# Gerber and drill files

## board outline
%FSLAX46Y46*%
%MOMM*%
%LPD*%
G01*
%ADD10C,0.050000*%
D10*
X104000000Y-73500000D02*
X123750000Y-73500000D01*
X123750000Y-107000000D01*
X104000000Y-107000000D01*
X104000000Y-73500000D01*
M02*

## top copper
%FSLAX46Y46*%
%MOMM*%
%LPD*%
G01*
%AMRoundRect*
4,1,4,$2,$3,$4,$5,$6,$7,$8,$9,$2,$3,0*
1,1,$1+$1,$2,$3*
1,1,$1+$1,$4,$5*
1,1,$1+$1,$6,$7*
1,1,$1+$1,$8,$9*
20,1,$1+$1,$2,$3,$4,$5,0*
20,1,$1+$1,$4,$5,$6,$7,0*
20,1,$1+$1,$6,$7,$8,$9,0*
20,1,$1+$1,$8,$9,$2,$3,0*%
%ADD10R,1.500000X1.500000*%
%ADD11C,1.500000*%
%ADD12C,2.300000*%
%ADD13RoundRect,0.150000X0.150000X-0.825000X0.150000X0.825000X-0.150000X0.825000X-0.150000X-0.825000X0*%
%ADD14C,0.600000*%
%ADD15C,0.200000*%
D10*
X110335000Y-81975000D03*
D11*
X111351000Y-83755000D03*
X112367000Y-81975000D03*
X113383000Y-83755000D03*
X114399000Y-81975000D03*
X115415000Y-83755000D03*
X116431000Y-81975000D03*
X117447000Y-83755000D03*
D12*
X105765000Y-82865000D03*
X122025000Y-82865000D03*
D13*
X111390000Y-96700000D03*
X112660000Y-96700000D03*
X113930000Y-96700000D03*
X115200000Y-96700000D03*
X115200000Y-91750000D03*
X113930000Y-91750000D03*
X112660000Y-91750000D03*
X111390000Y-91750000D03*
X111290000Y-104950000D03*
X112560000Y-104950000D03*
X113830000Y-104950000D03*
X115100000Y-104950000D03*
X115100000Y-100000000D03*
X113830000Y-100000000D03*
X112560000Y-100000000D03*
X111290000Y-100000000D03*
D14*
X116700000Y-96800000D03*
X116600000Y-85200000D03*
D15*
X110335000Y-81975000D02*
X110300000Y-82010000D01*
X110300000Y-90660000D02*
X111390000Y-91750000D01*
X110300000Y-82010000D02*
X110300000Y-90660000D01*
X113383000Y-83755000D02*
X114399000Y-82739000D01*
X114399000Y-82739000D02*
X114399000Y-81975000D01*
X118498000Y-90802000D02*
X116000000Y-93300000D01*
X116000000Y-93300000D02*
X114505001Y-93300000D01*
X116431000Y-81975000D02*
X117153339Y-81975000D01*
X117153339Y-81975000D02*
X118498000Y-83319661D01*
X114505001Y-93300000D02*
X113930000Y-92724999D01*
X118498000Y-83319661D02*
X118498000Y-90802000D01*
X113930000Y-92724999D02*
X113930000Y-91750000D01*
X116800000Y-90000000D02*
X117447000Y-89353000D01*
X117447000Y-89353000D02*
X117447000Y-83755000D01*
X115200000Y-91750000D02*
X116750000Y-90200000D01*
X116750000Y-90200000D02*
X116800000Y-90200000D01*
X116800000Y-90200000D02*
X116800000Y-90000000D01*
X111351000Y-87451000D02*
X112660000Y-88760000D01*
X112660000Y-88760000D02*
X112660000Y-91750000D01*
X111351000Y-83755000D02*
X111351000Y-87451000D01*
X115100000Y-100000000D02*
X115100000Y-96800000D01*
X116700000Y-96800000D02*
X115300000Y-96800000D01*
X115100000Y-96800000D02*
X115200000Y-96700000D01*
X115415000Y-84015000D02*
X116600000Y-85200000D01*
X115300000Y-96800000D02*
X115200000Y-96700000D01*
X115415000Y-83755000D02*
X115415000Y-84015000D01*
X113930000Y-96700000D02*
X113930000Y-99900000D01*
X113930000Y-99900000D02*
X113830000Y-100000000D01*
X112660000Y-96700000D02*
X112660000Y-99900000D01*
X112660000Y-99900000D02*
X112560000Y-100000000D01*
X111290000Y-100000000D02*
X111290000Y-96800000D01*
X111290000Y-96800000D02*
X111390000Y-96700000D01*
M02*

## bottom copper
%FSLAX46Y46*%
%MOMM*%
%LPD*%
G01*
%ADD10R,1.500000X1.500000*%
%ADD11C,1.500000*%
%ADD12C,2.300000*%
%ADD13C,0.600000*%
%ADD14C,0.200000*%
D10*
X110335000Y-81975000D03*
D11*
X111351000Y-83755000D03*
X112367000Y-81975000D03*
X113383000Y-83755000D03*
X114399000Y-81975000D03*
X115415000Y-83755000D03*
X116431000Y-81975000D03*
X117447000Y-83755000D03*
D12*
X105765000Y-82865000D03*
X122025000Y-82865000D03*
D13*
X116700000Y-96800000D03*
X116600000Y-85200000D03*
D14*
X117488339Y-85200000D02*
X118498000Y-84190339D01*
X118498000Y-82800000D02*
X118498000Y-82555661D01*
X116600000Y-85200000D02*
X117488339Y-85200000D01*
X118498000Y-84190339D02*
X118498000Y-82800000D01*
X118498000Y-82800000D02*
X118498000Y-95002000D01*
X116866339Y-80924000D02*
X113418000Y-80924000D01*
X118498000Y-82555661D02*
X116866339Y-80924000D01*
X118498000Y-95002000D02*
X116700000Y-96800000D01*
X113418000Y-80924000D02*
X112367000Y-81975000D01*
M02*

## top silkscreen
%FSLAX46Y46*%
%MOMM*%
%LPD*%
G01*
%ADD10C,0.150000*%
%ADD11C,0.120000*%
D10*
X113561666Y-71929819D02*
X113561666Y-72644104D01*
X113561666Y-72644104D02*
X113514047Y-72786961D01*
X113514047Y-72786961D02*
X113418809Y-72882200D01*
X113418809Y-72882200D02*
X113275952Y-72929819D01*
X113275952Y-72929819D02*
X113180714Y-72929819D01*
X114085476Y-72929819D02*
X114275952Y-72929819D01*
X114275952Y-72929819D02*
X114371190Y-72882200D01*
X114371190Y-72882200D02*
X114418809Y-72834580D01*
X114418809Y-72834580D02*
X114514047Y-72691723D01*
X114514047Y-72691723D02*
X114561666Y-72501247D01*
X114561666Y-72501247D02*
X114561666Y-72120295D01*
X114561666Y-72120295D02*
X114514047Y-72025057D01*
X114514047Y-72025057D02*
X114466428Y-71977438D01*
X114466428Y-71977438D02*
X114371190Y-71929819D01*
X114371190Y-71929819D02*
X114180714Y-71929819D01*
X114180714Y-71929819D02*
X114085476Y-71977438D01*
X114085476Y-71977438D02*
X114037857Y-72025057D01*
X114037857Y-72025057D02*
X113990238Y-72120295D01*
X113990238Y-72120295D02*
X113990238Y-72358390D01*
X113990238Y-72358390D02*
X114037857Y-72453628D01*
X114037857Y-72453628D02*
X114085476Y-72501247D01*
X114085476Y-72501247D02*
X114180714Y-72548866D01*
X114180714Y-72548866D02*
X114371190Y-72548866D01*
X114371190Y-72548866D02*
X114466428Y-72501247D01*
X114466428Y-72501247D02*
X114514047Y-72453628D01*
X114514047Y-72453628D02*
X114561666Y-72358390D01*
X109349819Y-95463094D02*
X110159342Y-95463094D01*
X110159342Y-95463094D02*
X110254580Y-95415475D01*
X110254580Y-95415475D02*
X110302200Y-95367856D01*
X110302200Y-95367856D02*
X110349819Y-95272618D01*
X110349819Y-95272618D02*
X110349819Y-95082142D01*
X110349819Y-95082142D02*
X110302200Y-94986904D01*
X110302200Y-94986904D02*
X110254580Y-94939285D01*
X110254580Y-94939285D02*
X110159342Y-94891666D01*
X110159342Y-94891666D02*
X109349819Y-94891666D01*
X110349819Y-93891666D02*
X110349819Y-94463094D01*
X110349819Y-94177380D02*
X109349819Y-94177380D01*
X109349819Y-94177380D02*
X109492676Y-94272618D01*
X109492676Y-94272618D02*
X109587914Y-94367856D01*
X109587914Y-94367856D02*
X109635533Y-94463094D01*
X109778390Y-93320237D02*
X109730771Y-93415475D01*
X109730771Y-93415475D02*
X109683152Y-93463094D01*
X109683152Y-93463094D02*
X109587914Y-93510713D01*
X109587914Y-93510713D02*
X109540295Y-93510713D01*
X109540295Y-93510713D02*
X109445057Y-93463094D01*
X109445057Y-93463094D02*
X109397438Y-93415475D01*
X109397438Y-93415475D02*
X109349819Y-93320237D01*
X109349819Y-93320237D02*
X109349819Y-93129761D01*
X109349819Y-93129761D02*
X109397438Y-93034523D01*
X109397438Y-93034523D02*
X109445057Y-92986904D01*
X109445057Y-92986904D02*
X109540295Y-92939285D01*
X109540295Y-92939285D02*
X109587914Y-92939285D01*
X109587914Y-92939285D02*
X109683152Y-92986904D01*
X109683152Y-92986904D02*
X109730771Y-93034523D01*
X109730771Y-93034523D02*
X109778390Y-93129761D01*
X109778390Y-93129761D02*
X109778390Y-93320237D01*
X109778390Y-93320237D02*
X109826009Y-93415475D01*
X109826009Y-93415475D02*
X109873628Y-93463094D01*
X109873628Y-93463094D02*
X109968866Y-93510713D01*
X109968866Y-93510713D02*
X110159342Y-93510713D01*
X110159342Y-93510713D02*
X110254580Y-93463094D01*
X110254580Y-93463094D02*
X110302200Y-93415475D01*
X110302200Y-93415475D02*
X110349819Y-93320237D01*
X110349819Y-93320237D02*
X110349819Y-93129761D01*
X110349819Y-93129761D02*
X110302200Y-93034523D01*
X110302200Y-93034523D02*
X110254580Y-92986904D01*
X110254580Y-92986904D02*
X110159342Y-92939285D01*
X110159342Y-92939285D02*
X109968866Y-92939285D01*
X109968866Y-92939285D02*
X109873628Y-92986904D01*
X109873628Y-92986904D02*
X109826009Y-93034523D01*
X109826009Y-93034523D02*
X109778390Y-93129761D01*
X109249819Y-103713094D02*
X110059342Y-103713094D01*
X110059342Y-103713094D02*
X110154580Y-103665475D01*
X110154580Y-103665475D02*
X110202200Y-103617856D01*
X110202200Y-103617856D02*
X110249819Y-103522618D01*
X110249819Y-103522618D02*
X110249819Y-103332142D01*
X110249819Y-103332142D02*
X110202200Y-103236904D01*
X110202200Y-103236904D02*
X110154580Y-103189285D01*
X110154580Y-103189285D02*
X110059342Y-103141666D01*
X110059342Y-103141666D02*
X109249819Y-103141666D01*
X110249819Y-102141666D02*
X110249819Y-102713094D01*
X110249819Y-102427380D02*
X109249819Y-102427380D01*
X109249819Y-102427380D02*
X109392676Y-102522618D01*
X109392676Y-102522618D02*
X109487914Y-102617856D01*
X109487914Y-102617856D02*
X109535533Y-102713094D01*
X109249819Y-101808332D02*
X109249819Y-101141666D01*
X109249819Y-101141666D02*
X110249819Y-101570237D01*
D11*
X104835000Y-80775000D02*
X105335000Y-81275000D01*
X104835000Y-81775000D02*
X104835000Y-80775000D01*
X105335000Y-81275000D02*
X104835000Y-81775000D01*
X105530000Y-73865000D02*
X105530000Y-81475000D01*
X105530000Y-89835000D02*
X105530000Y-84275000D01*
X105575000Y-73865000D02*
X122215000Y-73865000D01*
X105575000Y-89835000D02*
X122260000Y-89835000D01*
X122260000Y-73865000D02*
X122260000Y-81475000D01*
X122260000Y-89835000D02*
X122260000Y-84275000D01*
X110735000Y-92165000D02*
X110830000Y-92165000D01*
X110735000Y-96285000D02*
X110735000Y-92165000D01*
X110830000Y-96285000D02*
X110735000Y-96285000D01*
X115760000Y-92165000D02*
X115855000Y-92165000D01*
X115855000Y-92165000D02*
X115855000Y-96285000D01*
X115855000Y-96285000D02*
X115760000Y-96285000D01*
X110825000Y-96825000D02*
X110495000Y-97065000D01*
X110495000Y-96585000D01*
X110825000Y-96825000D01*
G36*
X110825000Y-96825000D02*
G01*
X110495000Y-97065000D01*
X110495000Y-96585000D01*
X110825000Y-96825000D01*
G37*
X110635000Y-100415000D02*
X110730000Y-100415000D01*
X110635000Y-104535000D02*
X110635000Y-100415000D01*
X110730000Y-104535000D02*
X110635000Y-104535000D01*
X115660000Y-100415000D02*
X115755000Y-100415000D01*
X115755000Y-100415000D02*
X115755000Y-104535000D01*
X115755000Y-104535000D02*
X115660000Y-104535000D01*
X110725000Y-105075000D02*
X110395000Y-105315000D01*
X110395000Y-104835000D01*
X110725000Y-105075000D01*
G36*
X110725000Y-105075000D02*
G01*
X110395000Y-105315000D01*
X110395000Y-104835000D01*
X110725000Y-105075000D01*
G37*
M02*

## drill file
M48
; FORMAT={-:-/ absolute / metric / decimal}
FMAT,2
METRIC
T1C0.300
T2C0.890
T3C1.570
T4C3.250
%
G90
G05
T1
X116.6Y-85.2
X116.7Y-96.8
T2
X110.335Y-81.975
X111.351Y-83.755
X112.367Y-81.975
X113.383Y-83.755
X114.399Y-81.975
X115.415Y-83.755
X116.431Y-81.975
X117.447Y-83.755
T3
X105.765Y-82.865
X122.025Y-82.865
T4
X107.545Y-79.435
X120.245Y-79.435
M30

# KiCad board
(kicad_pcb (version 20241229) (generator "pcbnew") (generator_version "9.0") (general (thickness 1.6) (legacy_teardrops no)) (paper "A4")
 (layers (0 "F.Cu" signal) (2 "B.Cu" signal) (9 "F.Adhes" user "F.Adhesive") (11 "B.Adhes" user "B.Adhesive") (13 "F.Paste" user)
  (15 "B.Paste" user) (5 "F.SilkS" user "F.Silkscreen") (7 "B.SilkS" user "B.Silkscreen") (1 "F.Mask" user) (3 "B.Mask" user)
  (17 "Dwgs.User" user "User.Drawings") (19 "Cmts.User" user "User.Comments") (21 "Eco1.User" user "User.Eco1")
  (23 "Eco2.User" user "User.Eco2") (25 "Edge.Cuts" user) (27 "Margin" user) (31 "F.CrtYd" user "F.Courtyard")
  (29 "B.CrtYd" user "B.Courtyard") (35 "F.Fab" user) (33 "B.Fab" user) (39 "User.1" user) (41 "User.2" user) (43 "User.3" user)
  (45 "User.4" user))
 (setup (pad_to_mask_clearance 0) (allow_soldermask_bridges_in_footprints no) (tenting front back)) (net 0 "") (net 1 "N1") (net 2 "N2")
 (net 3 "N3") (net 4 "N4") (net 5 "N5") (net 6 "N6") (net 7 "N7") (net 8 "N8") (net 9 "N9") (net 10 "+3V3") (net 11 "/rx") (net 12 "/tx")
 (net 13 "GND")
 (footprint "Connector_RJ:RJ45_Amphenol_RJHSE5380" (layer "F.Cu") (at 110.335 81.975)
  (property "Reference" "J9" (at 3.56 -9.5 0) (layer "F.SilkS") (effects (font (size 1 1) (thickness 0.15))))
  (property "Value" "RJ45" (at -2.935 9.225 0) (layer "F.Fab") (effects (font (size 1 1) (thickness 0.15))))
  (fp_line (start -5.5 -1.2) (end -5 -0.7) (stroke (width 0.12) (type solid)) (layer "F.SilkS"))
  (fp_line (start -5.5 -0.2) (end -5.5 -1.2) (stroke (width 0.12) (type solid)) (layer "F.SilkS"))
  (fp_line (start -5 -0.7) (end -5.5 -0.2) (stroke (width 0.12) (type solid)) (layer "F.SilkS"))
  (fp_line (start -4.805 -8.11) (end -4.805 -0.5) (stroke (width 0.12) (type solid)) (layer "F.SilkS"))
  (fp_line (start -4.805 7.86) (end -4.805 2.3) (stroke (width 0.12) (type solid)) (layer "F.SilkS"))
  (fp_line (start -4.76 -8.11) (end 11.88 -8.11) (stroke (width 0.12) (type solid)) (layer "F.SilkS"))
  (fp_line (start -4.76 7.86) (end 11.925 7.86) (stroke (width 0.12) (type solid)) (layer "F.SilkS"))
  (fp_line (start 11.925 -8.11) (end 11.925 -0.5) (stroke (width 0.12) (type solid)) (layer "F.SilkS"))
  (fp_line (start 11.925 7.86) (end 11.925 2.3) (stroke (width 0.12) (type solid)) (layer "F.SilkS"))
  (pad "" np_thru_hole circle (at -2.79 -2.54) (size 3.25 3.25) (drill 3.25) (layers "*.Cu" "*.Mask"))
  (pad "" np_thru_hole circle (at 9.91 -2.54) (size 3.25 3.25) (drill 3.25) (layers "*.Cu" "*.Mask"))
  (pad "1" thru_hole rect (at 0 0) (size 1.5 1.5) (drill 0.89) (layers "*.Cu" "*.Mask") (remove_unused_layers no) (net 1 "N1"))
  (pad "2" thru_hole circle (at 1.016 1.78) (size 1.5 1.5) (drill 0.89) (layers "*.Cu" "*.Mask") (remove_unused_layers no) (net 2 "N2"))
  (pad "3" thru_hole circle (at 2.032 0) (size 1.5 1.5) (drill 0.89) (layers "*.Cu" "*.Mask") (remove_unused_layers no) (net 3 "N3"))
  (pad "4" thru_hole circle (at 3.048 1.78) (size 1.5 1.5) (drill 0.89) (layers "*.Cu" "*.Mask") (remove_unused_layers no) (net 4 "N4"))
  (pad "5" thru_hole circle (at 4.064 0) (size 1.5 1.5) (drill 0.89) (layers "*.Cu" "*.Mask") (remove_unused_layers no) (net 4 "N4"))
  (pad "6" thru_hole circle (at 5.08 1.78) (size 1.5 1.5) (drill 0.89) (layers "*.Cu" "*.Mask") (remove_unused_layers no) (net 3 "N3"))
  (pad "7" thru_hole circle (at 6.096 0) (size 1.5 1.5) (drill 0.89) (layers "*.Cu" "*.Mask") (remove_unused_layers no) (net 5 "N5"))
  (pad "8" thru_hole circle (at 7.112 1.78) (size 1.5 1.5) (drill 0.89) (layers "*.Cu" "*.Mask") (remove_unused_layers no) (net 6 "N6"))
  (pad "SH" thru_hole circle (at -4.57 0.89) (size 2.3 2.3) (drill 1.57) (layers "*.Cu" "*.Mask") (remove_unused_layers no))
  (pad "SH" thru_hole circle (at 11.69 0.89) (size 2.3 2.3) (drill 1.57) (layers "*.Cu" "*.Mask") (remove_unused_layers no)))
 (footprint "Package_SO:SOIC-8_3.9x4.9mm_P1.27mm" (layer "F.Cu") (at 113.295 94.225 90)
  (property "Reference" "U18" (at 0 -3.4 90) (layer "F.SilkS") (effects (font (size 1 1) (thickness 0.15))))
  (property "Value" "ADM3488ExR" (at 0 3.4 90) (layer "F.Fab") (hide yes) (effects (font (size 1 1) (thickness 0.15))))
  (fp_line (start 2.06 -2.56) (end 2.06 -2.465) (stroke (width 0.12) (type solid)) (layer "F.SilkS"))
  (fp_line (start -2.06 -2.56) (end 2.06 -2.56) (stroke (width 0.12) (type solid)) (layer "F.SilkS"))
  (fp_line (start -2.06 -2.465) (end -2.06 -2.56) (stroke (width 0.12) (type solid)) (layer "F.SilkS"))
  (fp_line (start 2.06 2.465) (end 2.06 2.56) (stroke (width 0.12) (type solid)) (layer "F.SilkS"))
  (fp_line (start 2.06 2.56) (end -2.06 2.56) (stroke (width 0.12) (type solid)) (layer "F.SilkS"))
  (fp_line (start -2.06 2.56) (end -2.06 2.465) (stroke (width 0.12) (type solid)) (layer "F.SilkS"))
  (fp_poly (pts (xy -2.6 -2.47) (xy -2.84 -2.8) (xy -2.36 -2.8)) (stroke (width 0.12) (type solid)) (fill yes) (layer "F.SilkS"))
  (pad "1" smd roundrect (at -2.475 -1.905 90) (size 1.95 0.6) (layers "F.Cu" "F.Mask" "F.Paste") (roundrect_rratio 0.25) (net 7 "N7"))
  (pad "2" smd roundrect (at -2.475 -0.635 90) (size 1.95 0.6) (layers "F.Cu" "F.Mask" "F.Paste") (roundrect_rratio 0.25) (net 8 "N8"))
  (pad "3" smd roundrect (at -2.475 0.635 90) (size 1.95 0.6) (layers "F.Cu" "F.Mask" "F.Paste") (roundrect_rratio 0.25) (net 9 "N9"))
  (pad "4" smd roundrect (at -2.475 1.905 90) (size 1.95 0.6) (layers "F.Cu" "F.Mask" "F.Paste") (roundrect_rratio 0.25) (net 3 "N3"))
  (pad "5" smd roundrect (at 2.475 1.905 90) (size 1.95 0.6) (layers "F.Cu" "F.Mask" "F.Paste") (roundrect_rratio 0.25) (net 6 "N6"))
  (pad "6" smd roundrect (at 2.475 0.635 90) (size 1.95 0.6) (layers "F.Cu" "F.Mask" "F.Paste") (roundrect_rratio 0.25) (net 5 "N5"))
  (pad "7" smd roundrect (at 2.475 -0.635 90) (size 1.95 0.6) (layers "F.Cu" "F.Mask" "F.Paste") (roundrect_rratio 0.25) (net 2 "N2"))
  (pad "8" smd roundrect (at 2.475 -1.905 90) (size 1.95 0.6) (layers "F.Cu" "F.Mask" "F.Paste") (roundrect_rratio 0.25) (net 1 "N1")))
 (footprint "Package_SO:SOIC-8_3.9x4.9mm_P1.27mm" (layer "F.Cu") (at 113.195 102.475 90)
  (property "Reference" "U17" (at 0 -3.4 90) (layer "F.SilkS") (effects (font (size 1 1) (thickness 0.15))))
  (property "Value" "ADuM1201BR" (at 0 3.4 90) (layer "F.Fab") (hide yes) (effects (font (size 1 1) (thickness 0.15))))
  (fp_line (start 2.06 -2.56) (end 2.06 -2.465) (stroke (width 0.12) (type solid)) (layer "F.SilkS"))
  (fp_line (start -2.06 -2.56) (end 2.06 -2.56) (stroke (width 0.12) (type solid)) (layer "F.SilkS"))
  (fp_line (start -2.06 -2.465) (end -2.06 -2.56) (stroke (width 0.12) (type solid)) (layer "F.SilkS"))
  (fp_line (start 2.06 2.465) (end 2.06 2.56) (stroke (width 0.12) (type solid)) (layer "F.SilkS"))
  (fp_line (start 2.06 2.56) (end -2.06 2.56) (stroke (width 0.12) (type solid)) (layer "F.SilkS"))
  (fp_line (start -2.06 2.56) (end -2.06 2.465) (stroke (width 0.12) (type solid)) (layer "F.SilkS"))
  (fp_poly (pts (xy -2.6 -2.47) (xy -2.84 -2.8) (xy -2.36 -2.8)) (stroke (width 0.12) (type solid)) (fill yes) (layer "F.SilkS"))
  (pad "1" smd roundrect (at -2.475 -1.905 90) (size 1.95 0.6) (layers "F.Cu" "F.Mask" "F.Paste") (roundrect_rratio 0.25) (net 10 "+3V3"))
  (pad "2" smd roundrect (at -2.475 -0.635 90) (size 1.95 0.6) (layers "F.Cu" "F.Mask" "F.Paste") (roundrect_rratio 0.25) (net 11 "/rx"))
  (pad "3" smd roundrect (at -2.475 0.635 90) (size 1.95 0.6) (layers "F.Cu" "F.Mask" "F.Paste") (roundrect_rratio 0.25) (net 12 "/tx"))
  (pad "4" smd roundrect (at -2.475 1.905 90) (size 1.95 0.6) (layers "F.Cu" "F.Mask" "F.Paste") (roundrect_rratio 0.25) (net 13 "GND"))
  (pad "5" smd roundrect (at 2.475 1.905 90) (size 1.95 0.6) (layers "F.Cu" "F.Mask" "F.Paste") (roundrect_rratio 0.25) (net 3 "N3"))
  (pad "6" smd roundrect (at 2.475 0.635 90) (size 1.95 0.6) (layers "F.Cu" "F.Mask" "F.Paste") (roundrect_rratio 0.25) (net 9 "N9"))
  (pad "7" smd roundrect (at 2.475 -0.635 90) (size 1.95 0.6) (layers "F.Cu" "F.Mask" "F.Paste") (roundrect_rratio 0.25) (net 8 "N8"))
  (pad "8" smd roundrect (at 2.475 -1.905 90) (size 1.95 0.6) (layers "F.Cu" "F.Mask" "F.Paste") (roundrect_rratio 0.25) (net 7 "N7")))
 (gr_rect (start 104 73.5) (end 123.75 107) (stroke (width 0.05) (type default)) (fill no) (layer "Edge.Cuts"))
 (segment (start 110.335 81.975) (end 110.3 82.01) (width 0.2) (layer "F.Cu") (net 1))
 (segment (start 110.3 90.66) (end 111.39 91.75) (width 0.2) (layer "F.Cu") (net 1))
 (segment (start 110.3 82.01) (end 110.3 90.66) (width 0.2) (layer "F.Cu") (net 1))
 (segment (start 113.383 83.755) (end 114.399 82.739) (width 0.2) (layer "F.Cu") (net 4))
 (segment (start 114.399 82.739) (end 114.399 81.975) (width 0.2) (layer "F.Cu") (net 4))
 (segment (start 118.498 90.802) (end 116 93.3) (width 0.2) (layer "F.Cu") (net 5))
 (segment (start 116 93.3) (end 114.505001 93.3) (width 0.2) (layer "F.Cu") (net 5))
 (segment (start 116.431 81.975) (end 117.153339 81.975) (width 0.2) (layer "F.Cu") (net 5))
 (segment (start 117.153339 81.975) (end 118.498 83.319661) (width 0.2) (layer "F.Cu") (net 5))
 (segment (start 114.505001 93.3) (end 113.93 92.724999) (width 0.2) (layer "F.Cu") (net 5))
 (segment (start 118.498 83.319661) (end 118.498 90.802) (width 0.2) (layer "F.Cu") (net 5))
 (segment (start 113.93 92.724999) (end 113.93 91.75) (width 0.2) (layer "F.Cu") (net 5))
 (segment (start 116.8 90) (end 117.447 89.353) (width 0.2) (layer "F.Cu") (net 6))
 (segment (start 117.447 89.353) (end 117.447 83.755) (width 0.2) (layer "F.Cu") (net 6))
 (segment (start 115.2 91.75) (end 116.75 90.2) (width 0.2) (layer "F.Cu") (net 6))
 (segment (start 116.75 90.2) (end 116.8 90.2) (width 0.2) (layer "F.Cu") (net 6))
 (segment (start 116.8 90.2) (end 116.8 90) (width 0.2) (layer "F.Cu") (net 6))
 (segment (start 111.351 87.451) (end 112.66 88.76) (width 0.2) (layer "F.Cu") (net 2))
 (segment (start 112.66 88.76) (end 112.66 91.75) (width 0.2) (layer "F.Cu") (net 2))
 (segment (start 111.351 83.755) (end 111.351 87.451) (width 0.2) (layer "F.Cu") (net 2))
 (segment (start 115.1 100) (end 115.1 96.8) (width 0.2) (layer "F.Cu") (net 3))
 (segment (start 116.7 96.8) (end 115.3 96.8) (width 0.2) (layer "F.Cu") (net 3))
 (segment (start 115.1 96.8) (end 115.2 96.7) (width 0.2) (layer "F.Cu") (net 3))
 (segment (start 115.415 84.015) (end 116.6 85.2) (width 0.2) (layer "F.Cu") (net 3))
 (segment (start 115.3 96.8) (end 115.2 96.7) (width 0.2) (layer "F.Cu") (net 3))
 (segment (start 115.415 83.755) (end 115.415 84.015) (width 0.2) (layer "F.Cu") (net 3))
 (via (at 116.7 96.8) (size 0.6) (drill 0.3) (layers "F.Cu" "B.Cu") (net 3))
 (via (at 116.6 85.2) (size 0.6) (drill 0.3) (layers "F.Cu" "B.Cu") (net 3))
 (segment (start 117.488339 85.2) (end 118.498 84.190339) (width 0.2) (layer "B.Cu") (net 3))
 (segment (start 118.498 82.8) (end 118.498 82.555661) (width 0.2) (layer "B.Cu") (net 3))
 (segment (start 116.6 85.2) (end 117.488339 85.2) (width 0.2) (layer "B.Cu") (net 3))
 (segment (start 118.498 84.190339) (end 118.498 82.8) (width 0.2) (layer "B.Cu") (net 3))
 (segment (start 118.498 82.8) (end 118.498 95.002) (width 0.2) (layer "B.Cu") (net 3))
 (segment (start 116.866339 80.924) (end 113.418 80.924) (width 0.2) (layer "B.Cu") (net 3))
 (segment (start 118.498 82.555661) (end 116.866339 80.924) (width 0.2) (layer "B.Cu") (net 3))
 (segment (start 118.498 95.002) (end 116.7 96.8) (width 0.2) (layer "B.Cu") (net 3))
 (segment (start 113.418 80.924) (end 112.367 81.975) (width 0.2) (layer "B.Cu") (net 3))
 (segment (start 113.93 96.7) (end 113.93 99.9) (width 0.2) (layer "F.Cu") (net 9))
 (segment (start 113.93 99.9) (end 113.83 100) (width 0.2) (layer "F.Cu") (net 9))
 (segment (start 112.66 96.7) (end 112.66 99.9) (width 0.2) (layer "F.Cu") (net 8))
 (segment (start 112.66 99.9) (end 112.56 100) (width 0.2) (layer "F.Cu") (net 8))
 (segment (start 111.29 100) (end 111.29 96.8) (width 0.2) (layer "F.Cu") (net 7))
 (segment (start 111.29 96.8) (end 111.39 96.7) (width 0.2) (layer "F.Cu") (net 7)))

